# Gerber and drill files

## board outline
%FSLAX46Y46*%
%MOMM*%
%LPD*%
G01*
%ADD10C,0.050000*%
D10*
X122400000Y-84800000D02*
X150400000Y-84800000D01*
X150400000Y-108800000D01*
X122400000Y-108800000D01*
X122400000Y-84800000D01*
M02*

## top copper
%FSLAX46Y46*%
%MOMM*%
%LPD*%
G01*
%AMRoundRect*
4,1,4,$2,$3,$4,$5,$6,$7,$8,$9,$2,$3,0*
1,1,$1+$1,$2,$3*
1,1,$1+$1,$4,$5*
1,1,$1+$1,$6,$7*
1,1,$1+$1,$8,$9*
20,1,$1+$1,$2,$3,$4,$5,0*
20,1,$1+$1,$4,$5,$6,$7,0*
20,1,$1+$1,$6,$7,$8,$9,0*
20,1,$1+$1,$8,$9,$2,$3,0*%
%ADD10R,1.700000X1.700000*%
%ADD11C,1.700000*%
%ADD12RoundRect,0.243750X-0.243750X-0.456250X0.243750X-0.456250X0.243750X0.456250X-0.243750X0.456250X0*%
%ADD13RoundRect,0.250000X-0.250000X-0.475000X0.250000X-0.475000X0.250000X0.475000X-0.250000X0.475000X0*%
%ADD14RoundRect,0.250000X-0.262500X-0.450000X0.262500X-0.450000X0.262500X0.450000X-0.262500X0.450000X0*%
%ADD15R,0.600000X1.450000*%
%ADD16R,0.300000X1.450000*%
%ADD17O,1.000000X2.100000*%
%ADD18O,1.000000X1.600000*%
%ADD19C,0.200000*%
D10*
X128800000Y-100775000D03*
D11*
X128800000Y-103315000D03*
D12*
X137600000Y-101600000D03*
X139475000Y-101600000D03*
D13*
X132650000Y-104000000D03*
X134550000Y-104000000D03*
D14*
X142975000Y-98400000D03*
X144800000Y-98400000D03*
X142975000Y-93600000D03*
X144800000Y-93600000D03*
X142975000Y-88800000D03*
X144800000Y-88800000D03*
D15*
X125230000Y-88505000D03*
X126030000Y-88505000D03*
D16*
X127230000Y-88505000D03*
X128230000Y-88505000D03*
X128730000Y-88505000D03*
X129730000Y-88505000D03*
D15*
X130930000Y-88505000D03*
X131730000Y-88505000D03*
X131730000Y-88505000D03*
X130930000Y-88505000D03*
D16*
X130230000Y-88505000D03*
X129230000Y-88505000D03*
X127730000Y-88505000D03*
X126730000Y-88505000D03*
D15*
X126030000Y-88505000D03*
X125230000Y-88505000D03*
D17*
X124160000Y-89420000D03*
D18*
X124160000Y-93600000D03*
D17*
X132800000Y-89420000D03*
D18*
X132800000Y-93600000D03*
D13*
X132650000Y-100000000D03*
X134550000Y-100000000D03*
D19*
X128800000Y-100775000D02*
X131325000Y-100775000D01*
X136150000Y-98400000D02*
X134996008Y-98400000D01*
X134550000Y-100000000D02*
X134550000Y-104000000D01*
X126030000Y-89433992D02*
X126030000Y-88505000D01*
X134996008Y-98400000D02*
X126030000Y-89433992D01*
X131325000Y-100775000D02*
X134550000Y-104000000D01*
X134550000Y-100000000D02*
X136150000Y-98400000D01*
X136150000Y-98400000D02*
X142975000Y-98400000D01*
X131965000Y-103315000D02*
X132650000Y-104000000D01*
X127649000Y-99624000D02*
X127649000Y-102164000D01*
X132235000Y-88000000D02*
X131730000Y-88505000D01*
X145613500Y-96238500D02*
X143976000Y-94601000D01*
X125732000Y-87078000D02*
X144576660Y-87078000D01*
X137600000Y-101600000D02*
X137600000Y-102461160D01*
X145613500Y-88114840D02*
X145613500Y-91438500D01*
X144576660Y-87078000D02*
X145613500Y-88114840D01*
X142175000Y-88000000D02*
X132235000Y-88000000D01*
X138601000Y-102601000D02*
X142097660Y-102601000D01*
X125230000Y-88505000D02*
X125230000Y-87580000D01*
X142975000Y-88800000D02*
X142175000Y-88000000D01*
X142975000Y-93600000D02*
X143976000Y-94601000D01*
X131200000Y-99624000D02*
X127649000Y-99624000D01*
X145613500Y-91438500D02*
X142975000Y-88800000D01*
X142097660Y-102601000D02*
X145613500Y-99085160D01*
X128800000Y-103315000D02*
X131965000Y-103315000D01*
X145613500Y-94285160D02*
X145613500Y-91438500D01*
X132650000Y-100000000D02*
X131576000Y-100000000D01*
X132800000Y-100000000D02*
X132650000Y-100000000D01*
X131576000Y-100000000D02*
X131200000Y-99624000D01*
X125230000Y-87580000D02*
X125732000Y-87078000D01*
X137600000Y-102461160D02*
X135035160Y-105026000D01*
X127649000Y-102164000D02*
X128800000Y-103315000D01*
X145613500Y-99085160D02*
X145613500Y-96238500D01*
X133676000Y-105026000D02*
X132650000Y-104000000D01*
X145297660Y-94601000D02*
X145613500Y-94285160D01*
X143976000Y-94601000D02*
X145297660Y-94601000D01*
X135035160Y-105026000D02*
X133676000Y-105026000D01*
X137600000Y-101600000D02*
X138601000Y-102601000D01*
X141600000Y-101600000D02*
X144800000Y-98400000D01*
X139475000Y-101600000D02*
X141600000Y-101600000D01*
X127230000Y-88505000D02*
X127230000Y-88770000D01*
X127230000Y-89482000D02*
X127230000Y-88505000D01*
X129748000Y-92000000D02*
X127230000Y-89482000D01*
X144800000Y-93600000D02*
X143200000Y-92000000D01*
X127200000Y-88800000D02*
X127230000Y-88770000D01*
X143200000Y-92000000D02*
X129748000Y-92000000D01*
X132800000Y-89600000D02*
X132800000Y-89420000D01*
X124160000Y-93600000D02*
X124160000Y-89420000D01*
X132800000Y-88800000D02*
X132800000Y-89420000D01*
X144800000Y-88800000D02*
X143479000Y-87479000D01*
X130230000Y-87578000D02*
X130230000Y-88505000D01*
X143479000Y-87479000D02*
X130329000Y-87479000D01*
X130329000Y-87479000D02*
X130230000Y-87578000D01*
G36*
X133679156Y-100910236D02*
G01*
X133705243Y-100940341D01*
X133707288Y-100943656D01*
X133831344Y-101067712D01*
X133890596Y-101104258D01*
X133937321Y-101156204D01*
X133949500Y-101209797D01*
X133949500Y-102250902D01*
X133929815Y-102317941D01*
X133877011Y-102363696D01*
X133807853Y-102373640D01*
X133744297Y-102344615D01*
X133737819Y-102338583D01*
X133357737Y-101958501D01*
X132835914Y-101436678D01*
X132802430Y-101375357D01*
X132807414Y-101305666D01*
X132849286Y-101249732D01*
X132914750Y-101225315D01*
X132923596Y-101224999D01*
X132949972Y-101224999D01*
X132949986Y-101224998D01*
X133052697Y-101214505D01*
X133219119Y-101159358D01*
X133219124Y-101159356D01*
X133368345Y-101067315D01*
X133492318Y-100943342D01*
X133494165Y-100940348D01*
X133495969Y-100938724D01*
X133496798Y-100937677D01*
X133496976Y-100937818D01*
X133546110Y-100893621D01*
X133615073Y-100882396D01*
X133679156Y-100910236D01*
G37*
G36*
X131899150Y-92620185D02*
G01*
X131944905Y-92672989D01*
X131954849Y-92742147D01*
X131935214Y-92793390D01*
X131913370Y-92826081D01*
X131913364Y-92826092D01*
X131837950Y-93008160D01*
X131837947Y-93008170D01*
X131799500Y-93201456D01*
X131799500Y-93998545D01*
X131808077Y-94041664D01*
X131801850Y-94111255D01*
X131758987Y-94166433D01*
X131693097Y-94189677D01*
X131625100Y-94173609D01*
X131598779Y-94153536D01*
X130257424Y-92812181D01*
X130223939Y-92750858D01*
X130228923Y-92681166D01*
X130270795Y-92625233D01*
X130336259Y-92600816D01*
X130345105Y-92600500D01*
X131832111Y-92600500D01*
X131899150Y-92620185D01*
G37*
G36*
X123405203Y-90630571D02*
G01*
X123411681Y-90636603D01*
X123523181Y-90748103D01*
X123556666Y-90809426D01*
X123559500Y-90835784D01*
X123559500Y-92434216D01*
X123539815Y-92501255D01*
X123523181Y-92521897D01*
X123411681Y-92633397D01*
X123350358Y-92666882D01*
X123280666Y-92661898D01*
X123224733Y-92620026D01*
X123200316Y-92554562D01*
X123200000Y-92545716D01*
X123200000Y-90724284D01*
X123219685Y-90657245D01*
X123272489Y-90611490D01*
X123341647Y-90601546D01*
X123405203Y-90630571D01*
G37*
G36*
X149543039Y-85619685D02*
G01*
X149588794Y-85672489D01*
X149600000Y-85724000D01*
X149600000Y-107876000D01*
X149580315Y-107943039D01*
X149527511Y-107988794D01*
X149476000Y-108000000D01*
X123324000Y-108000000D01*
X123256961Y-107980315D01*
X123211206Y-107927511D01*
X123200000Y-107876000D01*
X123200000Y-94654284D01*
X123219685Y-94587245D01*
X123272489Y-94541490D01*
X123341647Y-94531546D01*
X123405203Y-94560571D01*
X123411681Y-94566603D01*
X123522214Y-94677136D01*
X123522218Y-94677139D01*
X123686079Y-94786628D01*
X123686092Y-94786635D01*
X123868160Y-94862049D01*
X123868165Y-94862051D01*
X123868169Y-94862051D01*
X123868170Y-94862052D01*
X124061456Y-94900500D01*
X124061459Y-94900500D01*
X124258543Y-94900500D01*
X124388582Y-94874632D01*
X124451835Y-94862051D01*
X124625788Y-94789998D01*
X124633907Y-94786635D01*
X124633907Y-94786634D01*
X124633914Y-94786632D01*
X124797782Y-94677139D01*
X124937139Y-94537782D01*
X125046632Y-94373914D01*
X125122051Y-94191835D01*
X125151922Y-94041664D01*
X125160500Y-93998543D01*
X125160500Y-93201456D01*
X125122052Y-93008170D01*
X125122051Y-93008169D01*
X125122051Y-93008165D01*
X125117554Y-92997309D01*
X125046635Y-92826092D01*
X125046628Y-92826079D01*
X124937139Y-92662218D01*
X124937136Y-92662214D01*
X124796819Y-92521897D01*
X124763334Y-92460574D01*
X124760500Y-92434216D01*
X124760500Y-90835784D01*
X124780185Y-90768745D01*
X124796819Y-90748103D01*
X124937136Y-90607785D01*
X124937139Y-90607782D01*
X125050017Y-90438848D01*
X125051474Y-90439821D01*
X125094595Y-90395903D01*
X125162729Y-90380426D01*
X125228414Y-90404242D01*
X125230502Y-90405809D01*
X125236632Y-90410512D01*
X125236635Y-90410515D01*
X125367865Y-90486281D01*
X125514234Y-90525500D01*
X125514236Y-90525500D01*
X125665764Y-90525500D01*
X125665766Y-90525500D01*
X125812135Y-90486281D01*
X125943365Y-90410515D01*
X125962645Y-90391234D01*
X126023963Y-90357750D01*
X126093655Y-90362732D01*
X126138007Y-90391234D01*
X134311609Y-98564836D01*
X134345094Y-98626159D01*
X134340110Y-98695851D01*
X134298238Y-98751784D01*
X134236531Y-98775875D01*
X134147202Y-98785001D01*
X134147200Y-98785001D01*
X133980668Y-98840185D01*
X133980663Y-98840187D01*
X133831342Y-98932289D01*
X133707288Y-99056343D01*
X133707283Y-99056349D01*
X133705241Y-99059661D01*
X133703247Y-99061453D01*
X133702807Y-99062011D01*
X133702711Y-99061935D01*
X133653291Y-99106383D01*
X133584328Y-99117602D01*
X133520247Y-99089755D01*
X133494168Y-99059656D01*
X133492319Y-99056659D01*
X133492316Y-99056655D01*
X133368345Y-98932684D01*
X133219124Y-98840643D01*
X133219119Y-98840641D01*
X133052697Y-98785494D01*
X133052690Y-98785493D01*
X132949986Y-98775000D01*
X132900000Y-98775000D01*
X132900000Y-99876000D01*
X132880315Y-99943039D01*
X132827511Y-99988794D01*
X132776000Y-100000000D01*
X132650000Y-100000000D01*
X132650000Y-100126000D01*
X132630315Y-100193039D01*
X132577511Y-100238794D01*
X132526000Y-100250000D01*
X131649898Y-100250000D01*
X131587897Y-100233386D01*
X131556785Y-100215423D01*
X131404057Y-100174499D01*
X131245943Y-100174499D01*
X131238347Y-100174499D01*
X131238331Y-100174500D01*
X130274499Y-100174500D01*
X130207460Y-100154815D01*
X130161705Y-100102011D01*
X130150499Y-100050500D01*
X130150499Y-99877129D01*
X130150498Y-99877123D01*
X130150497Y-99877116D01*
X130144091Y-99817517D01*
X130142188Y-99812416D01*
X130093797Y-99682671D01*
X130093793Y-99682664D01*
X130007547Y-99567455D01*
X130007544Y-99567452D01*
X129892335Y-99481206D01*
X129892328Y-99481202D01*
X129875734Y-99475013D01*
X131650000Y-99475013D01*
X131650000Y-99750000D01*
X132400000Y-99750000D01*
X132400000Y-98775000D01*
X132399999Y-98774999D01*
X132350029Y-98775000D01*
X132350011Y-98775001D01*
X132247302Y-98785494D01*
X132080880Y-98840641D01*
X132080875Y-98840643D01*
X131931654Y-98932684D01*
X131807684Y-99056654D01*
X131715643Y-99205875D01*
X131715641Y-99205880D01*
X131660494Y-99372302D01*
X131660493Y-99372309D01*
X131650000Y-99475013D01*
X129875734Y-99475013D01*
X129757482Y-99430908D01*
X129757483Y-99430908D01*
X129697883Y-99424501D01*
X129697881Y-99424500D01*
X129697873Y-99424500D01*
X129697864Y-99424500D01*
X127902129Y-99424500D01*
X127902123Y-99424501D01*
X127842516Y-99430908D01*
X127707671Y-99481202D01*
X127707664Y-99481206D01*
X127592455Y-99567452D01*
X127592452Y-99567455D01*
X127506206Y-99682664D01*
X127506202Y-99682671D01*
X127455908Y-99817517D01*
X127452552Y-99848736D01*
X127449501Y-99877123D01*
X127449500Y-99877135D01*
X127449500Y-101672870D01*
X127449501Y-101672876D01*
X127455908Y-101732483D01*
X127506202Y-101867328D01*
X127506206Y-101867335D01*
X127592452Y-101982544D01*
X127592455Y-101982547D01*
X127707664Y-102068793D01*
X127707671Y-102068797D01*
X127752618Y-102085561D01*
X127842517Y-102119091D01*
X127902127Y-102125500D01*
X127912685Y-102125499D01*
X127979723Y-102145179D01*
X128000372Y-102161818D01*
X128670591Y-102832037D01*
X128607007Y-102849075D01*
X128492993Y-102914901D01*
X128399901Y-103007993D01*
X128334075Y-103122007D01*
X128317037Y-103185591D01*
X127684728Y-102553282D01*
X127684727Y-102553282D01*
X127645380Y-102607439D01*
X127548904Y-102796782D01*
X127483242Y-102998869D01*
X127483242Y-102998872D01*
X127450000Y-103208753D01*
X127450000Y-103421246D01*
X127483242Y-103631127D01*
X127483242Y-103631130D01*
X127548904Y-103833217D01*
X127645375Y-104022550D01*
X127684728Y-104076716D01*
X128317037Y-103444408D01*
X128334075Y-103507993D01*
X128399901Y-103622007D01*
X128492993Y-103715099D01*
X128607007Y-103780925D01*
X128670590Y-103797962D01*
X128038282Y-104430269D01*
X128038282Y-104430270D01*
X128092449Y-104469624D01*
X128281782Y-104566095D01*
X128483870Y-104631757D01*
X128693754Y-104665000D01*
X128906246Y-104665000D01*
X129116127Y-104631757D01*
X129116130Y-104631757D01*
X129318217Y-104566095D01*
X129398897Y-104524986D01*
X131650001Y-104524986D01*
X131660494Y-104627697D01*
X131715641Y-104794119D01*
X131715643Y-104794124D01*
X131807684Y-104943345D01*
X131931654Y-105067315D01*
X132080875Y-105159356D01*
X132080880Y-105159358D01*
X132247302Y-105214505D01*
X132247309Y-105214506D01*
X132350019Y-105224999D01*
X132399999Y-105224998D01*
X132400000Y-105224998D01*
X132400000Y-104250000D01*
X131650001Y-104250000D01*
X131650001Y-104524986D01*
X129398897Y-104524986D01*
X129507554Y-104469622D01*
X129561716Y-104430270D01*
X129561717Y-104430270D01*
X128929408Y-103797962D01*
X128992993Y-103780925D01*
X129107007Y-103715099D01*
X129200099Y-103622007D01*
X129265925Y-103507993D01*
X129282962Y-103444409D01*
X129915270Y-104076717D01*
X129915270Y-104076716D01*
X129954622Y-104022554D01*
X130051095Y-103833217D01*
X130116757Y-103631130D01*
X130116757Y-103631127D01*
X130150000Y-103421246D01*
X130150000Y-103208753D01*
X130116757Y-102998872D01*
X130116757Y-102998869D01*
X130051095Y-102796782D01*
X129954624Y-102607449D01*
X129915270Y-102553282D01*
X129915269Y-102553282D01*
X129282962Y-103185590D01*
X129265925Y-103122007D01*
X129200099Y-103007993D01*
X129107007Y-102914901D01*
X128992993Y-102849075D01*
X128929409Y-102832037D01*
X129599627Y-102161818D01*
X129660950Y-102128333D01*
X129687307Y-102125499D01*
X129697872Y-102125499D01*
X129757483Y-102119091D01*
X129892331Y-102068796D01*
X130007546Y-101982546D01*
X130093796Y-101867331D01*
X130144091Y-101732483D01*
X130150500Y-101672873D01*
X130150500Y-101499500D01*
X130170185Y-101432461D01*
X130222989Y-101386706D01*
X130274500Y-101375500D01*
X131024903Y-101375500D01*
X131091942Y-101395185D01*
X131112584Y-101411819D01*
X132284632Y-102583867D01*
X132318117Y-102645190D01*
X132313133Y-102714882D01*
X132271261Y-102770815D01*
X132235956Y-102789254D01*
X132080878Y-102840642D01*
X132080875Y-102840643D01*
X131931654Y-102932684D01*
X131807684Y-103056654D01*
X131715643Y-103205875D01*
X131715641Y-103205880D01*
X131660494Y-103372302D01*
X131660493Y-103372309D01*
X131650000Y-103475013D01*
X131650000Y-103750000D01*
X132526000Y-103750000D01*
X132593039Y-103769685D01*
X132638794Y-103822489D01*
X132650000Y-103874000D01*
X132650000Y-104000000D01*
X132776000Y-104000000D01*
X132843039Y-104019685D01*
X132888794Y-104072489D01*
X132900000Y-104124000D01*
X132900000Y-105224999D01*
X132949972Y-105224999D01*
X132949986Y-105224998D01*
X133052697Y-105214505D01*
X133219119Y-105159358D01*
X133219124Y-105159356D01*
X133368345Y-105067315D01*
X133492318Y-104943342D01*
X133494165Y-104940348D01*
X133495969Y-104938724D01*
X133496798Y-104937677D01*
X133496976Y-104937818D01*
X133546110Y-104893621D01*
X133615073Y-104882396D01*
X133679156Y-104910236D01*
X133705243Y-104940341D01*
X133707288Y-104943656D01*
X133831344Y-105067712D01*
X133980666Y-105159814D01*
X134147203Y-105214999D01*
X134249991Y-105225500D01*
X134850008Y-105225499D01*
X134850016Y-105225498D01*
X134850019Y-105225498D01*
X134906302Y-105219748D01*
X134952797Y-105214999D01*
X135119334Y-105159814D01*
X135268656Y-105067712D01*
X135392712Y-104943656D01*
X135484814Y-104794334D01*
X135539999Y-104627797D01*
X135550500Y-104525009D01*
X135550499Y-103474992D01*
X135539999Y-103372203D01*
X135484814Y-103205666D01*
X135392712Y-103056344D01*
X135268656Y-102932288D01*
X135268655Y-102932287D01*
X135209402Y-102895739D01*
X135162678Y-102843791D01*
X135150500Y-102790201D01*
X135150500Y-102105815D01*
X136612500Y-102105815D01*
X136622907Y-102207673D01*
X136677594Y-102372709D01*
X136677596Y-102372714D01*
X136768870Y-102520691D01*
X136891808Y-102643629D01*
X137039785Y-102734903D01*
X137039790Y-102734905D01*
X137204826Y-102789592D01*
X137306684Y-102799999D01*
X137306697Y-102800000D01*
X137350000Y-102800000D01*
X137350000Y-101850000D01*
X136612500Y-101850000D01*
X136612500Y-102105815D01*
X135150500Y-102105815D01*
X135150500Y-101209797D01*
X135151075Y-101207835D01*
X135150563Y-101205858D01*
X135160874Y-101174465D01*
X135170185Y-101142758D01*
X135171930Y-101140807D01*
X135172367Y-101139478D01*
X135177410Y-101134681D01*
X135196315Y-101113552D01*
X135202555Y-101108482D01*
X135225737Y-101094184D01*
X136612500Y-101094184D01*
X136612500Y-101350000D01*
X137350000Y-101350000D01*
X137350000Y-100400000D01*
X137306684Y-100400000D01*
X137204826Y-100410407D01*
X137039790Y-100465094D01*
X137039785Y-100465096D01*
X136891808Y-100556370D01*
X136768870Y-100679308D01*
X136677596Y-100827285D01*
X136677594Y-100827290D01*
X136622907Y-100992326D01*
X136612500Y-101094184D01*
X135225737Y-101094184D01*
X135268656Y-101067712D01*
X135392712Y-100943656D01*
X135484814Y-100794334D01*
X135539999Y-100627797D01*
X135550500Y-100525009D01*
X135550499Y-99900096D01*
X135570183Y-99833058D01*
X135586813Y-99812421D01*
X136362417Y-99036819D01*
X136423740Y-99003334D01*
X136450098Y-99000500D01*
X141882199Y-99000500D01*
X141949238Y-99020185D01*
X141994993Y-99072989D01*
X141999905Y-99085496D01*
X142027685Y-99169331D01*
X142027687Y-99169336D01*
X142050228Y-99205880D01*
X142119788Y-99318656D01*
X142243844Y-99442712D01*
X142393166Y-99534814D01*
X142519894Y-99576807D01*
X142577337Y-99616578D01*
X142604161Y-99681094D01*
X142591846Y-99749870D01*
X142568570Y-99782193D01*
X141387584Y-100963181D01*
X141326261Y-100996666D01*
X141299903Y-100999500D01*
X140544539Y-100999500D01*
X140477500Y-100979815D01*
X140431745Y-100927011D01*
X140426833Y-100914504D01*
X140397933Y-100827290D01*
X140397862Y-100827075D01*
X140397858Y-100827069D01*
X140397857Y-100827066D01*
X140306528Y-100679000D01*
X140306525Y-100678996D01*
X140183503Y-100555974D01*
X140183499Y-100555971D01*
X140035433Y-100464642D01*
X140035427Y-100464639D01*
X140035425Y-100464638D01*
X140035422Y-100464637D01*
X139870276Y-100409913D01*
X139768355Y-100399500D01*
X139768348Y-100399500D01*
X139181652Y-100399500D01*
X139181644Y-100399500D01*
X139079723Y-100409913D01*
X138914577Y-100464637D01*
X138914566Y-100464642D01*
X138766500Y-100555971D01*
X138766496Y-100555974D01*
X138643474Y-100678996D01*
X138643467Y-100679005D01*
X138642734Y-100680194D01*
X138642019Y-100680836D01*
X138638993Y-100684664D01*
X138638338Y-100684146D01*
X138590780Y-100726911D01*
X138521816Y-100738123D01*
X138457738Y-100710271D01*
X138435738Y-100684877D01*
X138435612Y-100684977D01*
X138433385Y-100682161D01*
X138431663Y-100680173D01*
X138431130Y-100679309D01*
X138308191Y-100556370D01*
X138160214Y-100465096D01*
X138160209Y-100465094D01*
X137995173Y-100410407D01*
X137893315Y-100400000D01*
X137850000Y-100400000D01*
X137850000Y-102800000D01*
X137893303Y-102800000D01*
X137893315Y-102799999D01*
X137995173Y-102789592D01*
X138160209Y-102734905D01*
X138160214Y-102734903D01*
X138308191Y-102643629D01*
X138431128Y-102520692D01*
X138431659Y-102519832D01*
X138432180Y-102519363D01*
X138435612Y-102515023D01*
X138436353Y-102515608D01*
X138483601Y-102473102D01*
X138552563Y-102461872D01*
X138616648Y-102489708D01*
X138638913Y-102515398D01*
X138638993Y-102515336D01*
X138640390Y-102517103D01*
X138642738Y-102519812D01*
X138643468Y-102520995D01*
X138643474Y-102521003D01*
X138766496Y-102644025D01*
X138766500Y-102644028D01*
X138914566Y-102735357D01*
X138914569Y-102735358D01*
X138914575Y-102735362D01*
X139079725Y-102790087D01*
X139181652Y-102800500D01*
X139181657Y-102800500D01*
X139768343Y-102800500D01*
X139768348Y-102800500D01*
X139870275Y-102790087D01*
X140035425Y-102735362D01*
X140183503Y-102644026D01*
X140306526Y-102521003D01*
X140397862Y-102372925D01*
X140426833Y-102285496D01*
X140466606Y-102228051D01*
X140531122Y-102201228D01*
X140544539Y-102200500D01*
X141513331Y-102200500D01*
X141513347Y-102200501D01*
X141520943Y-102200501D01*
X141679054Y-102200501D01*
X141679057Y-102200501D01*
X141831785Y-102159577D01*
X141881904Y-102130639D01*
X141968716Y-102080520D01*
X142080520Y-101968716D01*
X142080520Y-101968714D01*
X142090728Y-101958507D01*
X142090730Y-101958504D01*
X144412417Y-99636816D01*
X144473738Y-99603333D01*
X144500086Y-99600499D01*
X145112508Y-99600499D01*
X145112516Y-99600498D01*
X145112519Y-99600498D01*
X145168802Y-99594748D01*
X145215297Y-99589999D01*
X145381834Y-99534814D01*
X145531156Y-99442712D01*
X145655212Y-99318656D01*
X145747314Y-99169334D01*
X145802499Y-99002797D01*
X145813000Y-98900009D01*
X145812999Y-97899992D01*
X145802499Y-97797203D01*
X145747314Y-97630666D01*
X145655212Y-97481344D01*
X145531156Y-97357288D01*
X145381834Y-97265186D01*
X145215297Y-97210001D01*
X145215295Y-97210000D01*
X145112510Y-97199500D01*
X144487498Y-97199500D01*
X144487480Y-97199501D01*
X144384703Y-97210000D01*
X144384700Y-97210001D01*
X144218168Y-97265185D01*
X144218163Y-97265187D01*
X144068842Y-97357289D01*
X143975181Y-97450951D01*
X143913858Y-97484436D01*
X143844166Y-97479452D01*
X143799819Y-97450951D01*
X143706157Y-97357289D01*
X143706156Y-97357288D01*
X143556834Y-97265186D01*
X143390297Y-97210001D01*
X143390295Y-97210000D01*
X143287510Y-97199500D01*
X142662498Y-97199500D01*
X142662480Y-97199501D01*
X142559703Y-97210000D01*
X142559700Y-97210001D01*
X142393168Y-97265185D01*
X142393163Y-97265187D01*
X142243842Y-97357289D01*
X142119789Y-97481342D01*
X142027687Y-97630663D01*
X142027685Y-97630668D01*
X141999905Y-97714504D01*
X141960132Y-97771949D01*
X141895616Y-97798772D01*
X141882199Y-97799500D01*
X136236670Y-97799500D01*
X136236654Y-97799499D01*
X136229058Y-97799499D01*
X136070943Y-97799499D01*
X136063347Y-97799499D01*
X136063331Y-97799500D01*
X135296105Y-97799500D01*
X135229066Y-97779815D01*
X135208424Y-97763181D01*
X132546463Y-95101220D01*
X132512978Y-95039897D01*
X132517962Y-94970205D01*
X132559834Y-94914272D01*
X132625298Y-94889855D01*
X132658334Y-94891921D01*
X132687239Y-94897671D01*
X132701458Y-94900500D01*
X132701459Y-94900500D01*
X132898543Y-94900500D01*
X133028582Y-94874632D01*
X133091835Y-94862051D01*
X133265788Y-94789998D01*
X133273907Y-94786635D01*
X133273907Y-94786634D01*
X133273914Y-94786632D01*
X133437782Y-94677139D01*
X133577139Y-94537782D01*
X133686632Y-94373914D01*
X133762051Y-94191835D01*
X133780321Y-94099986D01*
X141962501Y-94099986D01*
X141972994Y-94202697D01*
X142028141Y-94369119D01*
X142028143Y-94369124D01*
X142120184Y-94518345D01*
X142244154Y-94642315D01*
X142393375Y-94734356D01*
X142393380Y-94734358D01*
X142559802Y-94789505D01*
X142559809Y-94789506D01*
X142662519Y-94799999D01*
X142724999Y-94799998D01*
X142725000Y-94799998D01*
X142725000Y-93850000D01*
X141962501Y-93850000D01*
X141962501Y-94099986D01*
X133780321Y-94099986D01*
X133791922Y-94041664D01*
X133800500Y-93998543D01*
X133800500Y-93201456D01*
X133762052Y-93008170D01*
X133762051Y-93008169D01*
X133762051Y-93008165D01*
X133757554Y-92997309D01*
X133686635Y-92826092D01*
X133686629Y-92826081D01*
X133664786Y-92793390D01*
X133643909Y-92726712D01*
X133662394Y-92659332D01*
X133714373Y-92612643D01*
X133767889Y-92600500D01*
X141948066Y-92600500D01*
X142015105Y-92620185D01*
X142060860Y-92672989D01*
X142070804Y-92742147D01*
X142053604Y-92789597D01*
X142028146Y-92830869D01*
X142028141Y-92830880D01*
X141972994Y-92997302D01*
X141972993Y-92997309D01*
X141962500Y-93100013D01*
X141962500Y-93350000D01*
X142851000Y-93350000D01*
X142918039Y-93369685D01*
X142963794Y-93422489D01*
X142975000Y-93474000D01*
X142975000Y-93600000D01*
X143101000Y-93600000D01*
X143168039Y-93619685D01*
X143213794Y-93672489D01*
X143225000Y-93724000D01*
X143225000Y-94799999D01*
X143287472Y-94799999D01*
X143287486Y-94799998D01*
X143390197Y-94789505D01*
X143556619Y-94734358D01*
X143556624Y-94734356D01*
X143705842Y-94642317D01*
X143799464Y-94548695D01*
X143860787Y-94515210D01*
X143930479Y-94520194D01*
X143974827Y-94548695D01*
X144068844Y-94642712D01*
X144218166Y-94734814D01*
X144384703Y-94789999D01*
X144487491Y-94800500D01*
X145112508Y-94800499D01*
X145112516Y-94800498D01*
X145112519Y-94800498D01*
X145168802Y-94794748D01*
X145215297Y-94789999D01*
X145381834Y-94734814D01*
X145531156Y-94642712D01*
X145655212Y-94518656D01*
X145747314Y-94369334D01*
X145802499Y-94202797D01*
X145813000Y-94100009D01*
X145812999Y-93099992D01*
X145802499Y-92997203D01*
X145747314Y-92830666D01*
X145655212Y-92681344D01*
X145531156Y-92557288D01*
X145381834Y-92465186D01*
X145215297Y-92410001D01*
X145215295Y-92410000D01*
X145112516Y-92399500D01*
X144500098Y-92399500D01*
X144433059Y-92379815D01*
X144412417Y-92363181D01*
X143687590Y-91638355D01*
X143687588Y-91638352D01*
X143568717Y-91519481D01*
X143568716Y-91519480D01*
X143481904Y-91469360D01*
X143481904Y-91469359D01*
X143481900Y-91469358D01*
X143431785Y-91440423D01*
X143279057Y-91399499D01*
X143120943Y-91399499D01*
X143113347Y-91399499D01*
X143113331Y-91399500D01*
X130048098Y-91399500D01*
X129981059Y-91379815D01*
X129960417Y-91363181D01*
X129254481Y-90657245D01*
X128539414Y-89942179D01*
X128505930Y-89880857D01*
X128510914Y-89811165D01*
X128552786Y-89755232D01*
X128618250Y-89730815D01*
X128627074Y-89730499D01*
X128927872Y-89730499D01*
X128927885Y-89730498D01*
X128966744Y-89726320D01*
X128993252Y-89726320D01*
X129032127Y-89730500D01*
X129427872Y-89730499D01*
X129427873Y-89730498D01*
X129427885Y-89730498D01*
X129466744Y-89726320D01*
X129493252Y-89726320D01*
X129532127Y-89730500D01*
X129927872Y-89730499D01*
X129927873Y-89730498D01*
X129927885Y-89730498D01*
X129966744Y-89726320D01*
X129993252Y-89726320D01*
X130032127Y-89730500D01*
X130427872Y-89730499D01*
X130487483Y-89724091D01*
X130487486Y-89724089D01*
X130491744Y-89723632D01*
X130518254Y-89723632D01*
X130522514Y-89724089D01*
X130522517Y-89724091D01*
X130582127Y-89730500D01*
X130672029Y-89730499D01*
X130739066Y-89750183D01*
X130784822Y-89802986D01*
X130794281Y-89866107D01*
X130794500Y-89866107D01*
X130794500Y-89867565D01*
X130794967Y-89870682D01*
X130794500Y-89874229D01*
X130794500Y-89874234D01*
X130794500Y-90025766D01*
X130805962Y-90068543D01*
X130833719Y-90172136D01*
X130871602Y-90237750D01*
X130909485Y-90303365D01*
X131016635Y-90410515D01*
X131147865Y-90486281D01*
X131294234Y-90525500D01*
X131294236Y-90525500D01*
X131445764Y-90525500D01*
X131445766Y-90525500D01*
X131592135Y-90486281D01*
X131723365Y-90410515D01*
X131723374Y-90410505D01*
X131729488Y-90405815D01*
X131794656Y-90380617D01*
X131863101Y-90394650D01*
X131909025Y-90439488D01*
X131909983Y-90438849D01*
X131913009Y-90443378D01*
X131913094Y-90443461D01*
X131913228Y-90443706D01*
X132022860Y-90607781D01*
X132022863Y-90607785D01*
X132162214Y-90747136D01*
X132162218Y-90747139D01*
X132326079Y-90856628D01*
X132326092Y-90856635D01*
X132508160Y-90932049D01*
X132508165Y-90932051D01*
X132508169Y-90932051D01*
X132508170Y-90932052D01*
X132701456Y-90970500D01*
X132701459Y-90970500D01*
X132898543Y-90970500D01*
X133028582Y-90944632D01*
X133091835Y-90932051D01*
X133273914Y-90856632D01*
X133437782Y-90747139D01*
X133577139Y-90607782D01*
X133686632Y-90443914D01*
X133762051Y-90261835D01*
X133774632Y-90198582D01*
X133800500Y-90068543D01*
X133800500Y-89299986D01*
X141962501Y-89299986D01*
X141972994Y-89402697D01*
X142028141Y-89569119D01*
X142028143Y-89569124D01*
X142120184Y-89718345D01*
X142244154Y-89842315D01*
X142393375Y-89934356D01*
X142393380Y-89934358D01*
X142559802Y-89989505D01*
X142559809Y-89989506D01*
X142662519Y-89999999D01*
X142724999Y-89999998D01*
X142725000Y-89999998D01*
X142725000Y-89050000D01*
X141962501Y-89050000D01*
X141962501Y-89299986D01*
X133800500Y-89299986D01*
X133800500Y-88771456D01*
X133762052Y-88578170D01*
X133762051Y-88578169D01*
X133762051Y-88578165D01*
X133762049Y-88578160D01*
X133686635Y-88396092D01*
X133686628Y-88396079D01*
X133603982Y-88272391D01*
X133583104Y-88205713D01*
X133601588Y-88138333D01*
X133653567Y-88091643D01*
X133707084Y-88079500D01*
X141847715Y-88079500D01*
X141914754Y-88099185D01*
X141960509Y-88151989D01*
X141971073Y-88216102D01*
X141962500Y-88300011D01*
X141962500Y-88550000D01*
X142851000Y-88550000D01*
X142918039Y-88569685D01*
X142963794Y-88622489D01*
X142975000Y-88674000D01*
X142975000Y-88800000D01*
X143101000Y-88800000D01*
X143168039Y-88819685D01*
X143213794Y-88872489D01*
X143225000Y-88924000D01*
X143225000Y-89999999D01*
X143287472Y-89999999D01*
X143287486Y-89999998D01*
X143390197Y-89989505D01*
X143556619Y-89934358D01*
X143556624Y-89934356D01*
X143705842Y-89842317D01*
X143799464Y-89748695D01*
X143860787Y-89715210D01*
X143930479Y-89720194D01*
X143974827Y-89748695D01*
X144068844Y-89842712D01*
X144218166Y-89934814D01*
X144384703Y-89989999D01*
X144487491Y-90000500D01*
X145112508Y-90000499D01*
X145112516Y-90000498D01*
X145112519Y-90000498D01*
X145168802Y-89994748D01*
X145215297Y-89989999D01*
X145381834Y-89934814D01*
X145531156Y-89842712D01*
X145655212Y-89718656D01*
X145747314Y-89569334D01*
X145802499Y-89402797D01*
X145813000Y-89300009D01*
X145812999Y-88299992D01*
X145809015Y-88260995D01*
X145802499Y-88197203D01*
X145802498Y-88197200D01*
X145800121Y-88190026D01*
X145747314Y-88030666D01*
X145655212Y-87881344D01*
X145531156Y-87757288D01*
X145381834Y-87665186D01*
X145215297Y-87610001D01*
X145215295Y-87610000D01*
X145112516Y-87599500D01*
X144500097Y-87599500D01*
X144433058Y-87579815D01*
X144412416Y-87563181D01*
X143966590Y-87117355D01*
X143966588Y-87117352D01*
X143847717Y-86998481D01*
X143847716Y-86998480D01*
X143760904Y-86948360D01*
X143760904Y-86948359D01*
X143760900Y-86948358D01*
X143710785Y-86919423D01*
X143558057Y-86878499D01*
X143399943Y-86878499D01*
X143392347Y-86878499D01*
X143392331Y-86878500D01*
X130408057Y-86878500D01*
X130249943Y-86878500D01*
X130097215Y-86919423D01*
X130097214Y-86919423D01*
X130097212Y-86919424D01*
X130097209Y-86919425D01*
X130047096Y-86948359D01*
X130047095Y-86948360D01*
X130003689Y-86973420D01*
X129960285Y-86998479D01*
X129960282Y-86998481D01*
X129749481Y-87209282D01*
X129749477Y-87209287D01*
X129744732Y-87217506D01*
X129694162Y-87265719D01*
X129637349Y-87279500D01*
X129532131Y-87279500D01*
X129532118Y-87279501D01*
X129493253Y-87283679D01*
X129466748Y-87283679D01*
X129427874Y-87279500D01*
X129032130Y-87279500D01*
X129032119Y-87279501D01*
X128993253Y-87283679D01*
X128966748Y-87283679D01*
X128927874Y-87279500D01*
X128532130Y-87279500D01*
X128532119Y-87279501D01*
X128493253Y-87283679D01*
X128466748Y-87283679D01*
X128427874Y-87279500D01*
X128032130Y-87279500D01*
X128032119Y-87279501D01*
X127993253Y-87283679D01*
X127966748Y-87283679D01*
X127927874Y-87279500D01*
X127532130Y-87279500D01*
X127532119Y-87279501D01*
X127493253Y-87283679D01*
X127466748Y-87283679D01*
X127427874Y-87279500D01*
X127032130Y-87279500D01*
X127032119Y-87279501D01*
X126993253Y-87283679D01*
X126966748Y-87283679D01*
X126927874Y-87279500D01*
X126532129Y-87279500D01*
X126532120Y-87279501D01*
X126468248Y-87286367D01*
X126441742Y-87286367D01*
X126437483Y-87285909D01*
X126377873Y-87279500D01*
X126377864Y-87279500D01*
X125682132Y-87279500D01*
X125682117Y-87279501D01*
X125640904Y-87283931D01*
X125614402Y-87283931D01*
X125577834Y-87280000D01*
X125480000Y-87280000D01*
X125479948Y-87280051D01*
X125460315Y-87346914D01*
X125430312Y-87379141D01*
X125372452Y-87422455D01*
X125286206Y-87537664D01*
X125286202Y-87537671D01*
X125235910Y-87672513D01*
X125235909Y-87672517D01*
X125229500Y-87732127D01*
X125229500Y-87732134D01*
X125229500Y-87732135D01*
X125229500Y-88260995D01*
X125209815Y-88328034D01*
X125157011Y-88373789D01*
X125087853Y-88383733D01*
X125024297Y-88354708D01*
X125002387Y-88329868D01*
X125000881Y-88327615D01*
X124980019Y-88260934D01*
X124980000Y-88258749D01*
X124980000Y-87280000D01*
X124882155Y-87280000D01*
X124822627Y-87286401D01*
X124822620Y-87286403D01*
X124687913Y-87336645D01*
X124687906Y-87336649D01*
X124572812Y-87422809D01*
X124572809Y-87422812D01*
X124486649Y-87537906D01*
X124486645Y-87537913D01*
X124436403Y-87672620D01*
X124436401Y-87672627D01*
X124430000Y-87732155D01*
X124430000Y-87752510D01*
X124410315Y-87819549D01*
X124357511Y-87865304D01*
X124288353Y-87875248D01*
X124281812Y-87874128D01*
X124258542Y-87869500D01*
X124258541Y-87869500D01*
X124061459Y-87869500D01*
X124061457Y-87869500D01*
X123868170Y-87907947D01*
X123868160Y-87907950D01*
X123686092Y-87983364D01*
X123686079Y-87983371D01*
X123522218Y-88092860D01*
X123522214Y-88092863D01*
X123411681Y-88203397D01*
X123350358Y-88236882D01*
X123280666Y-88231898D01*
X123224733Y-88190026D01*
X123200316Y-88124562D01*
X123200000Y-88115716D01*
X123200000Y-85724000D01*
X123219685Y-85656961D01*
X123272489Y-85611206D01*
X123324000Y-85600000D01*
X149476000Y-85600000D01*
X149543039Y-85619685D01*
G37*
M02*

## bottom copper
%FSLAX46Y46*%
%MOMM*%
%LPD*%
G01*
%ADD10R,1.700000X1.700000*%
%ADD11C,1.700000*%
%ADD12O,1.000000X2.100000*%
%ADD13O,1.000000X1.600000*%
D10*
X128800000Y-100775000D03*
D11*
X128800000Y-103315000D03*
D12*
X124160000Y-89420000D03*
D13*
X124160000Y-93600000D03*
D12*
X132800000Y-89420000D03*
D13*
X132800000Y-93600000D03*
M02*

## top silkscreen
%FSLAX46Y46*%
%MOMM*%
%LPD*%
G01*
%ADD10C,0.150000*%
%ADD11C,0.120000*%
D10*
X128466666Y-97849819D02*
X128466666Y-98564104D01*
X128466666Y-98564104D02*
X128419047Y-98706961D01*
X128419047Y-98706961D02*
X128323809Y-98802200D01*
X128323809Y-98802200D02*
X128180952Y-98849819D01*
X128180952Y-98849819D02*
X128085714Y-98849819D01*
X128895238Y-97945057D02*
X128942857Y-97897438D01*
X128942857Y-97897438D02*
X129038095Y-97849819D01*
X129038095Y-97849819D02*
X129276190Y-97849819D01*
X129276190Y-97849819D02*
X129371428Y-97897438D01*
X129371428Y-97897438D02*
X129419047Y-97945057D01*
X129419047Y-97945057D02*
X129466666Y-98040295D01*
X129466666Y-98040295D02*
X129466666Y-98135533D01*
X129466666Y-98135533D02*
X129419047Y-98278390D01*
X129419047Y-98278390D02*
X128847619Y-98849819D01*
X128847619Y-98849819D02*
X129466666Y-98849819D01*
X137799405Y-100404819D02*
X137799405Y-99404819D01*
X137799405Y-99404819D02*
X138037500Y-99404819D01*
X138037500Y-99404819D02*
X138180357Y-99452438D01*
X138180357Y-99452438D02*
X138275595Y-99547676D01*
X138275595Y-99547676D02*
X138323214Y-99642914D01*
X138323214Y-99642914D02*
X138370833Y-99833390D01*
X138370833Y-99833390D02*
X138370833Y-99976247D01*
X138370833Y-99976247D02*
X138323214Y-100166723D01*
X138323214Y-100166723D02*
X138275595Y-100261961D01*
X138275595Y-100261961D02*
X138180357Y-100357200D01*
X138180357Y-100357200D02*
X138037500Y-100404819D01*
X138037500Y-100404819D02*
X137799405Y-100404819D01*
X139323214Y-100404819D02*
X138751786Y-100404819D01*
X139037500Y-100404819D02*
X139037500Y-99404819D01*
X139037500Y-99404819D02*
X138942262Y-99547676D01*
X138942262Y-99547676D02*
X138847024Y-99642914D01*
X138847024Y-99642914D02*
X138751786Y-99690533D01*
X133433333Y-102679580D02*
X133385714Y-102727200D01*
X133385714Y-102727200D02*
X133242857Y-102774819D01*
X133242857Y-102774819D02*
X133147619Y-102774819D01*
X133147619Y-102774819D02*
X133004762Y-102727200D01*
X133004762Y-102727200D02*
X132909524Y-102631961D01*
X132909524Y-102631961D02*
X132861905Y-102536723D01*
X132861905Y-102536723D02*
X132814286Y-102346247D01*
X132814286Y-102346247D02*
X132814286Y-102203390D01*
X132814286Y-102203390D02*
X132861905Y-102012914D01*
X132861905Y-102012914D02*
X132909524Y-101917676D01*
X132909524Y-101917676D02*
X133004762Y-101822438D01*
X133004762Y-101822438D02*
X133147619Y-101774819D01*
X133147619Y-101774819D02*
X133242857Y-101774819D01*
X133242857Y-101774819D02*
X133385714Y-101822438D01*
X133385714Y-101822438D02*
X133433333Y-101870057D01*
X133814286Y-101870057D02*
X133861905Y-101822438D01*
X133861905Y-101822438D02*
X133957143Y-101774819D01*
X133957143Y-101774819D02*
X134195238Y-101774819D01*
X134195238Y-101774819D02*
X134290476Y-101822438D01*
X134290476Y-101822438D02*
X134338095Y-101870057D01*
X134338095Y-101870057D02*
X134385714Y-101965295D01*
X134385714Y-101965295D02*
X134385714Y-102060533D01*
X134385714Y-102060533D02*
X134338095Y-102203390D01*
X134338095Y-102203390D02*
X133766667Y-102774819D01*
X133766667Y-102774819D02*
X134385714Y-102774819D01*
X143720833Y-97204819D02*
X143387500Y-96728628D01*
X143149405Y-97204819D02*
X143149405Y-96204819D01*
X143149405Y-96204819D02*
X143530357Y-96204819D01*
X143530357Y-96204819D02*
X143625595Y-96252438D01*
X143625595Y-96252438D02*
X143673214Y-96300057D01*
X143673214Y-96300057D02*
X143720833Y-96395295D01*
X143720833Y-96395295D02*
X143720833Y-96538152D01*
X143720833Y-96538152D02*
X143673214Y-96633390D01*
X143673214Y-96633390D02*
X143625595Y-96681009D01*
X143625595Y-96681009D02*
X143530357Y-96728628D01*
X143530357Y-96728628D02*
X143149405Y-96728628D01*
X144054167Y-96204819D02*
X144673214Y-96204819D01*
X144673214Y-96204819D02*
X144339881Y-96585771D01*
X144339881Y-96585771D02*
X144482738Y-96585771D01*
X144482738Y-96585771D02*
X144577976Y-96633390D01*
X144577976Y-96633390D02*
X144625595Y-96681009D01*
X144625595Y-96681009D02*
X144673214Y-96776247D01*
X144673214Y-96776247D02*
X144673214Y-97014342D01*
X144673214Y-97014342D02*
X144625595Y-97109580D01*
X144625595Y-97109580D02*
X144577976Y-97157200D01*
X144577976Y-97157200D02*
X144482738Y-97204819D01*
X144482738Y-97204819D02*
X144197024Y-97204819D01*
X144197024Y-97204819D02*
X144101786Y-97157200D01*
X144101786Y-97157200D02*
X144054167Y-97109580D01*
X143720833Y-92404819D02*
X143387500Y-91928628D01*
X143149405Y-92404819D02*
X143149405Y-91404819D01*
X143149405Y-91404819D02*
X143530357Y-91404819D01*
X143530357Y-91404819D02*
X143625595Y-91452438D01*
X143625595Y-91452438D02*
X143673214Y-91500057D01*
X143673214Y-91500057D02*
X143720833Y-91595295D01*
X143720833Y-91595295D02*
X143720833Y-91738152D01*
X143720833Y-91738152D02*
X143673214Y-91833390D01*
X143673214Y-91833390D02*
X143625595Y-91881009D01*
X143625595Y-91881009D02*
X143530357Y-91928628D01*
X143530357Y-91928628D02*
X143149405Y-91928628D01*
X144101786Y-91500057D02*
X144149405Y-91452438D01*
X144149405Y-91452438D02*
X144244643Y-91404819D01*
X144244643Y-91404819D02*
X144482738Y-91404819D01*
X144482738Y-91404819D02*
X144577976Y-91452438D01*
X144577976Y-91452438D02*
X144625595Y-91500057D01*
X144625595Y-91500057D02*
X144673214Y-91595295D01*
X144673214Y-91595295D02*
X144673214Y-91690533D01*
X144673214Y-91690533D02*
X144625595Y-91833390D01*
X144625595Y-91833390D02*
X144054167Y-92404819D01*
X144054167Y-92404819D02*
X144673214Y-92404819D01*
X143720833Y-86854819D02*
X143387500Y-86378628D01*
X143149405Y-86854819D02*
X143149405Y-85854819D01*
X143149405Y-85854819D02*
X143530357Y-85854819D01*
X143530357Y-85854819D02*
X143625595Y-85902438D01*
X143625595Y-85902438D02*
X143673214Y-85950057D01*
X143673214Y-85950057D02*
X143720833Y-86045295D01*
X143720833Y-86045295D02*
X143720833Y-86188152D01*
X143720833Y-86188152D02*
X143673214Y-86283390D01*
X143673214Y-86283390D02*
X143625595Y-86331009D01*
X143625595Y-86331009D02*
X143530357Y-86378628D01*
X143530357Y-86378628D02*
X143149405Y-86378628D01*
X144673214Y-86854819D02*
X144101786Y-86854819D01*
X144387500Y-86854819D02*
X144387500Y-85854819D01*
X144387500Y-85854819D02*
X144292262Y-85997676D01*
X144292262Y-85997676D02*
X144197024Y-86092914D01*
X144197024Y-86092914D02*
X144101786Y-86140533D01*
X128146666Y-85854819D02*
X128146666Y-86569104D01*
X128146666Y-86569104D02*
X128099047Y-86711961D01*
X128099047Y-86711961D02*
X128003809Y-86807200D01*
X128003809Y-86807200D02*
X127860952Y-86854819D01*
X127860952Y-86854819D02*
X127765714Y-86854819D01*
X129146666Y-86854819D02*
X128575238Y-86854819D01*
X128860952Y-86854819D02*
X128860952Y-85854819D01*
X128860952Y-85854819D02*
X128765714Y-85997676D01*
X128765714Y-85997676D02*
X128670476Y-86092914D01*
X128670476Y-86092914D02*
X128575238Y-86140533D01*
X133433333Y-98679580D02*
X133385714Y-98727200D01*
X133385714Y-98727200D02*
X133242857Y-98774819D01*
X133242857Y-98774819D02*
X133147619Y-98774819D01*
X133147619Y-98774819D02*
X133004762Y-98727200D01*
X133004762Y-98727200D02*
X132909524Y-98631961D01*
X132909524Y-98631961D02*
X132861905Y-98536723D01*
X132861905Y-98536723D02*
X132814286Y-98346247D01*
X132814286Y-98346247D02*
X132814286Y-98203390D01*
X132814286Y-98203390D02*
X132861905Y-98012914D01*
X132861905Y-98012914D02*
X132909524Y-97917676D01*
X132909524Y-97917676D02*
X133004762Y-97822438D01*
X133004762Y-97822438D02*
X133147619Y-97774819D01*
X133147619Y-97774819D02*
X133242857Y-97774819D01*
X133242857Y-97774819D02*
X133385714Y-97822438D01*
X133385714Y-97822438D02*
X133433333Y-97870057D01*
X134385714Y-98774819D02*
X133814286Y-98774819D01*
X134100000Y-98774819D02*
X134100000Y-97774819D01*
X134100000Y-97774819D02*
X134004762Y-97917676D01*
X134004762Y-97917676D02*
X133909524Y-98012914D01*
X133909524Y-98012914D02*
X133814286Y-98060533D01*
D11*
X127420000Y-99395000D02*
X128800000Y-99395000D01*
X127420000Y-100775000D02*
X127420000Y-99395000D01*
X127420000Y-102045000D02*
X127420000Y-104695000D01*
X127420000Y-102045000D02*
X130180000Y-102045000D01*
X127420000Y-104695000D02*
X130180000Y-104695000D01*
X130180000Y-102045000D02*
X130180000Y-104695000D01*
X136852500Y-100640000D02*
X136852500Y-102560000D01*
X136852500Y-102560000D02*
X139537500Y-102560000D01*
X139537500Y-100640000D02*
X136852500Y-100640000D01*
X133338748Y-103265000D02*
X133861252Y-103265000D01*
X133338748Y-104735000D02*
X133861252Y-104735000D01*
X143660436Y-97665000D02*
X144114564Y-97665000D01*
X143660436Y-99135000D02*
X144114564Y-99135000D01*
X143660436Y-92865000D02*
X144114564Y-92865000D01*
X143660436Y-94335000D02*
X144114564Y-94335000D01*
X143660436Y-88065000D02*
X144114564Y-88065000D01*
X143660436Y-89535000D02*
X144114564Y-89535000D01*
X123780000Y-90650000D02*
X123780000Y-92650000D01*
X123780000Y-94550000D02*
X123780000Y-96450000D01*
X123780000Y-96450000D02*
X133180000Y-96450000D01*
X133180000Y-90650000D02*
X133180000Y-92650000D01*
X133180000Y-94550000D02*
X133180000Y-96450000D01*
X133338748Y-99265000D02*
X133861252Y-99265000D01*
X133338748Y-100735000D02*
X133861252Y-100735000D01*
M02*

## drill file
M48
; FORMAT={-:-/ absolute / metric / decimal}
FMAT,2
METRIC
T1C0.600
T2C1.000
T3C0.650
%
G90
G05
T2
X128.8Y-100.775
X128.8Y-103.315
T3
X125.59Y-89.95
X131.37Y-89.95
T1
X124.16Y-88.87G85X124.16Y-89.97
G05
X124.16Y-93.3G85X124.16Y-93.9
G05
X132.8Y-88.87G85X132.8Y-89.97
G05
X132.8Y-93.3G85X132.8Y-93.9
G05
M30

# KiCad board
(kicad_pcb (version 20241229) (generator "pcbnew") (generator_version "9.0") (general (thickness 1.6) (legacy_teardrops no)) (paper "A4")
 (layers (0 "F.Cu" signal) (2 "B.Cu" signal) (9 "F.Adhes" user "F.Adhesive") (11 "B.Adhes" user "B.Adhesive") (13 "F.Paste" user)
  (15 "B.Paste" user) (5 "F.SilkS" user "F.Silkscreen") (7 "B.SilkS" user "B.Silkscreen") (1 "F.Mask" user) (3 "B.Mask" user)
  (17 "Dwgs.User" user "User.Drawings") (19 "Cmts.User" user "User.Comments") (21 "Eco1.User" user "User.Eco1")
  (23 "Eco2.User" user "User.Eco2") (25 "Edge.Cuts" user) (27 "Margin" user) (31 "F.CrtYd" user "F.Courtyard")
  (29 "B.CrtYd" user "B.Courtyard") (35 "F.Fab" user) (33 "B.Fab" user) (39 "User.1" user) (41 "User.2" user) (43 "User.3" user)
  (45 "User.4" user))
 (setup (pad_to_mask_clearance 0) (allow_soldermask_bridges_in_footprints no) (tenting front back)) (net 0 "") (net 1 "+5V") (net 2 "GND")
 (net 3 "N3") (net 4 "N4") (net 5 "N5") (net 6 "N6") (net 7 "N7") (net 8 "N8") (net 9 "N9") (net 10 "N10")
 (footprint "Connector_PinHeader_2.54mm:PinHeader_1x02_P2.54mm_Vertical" (layer "F.Cu") (at 128.8 100.775)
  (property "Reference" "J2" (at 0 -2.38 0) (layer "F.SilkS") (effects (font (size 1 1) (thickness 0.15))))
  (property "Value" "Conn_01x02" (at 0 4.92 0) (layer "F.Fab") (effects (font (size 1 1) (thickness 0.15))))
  (fp_line (start -1.38 -1.38) (end 0 -1.38) (stroke (width 0.12) (type solid)) (layer "F.SilkS"))
  (fp_line (start -1.38 0) (end -1.38 -1.38) (stroke (width 0.12) (type solid)) (layer "F.SilkS"))
  (fp_line (start -1.38 1.27) (end -1.38 3.92) (stroke (width 0.12) (type solid)) (layer "F.SilkS"))
  (fp_line (start -1.38 1.27) (end 1.38 1.27) (stroke (width 0.12) (type solid)) (layer "F.SilkS"))
  (fp_line (start -1.38 3.92) (end 1.38 3.92) (stroke (width 0.12) (type solid)) (layer "F.SilkS"))
  (fp_line (start 1.38 1.27) (end 1.38 3.92) (stroke (width 0.12) (type solid)) (layer "F.SilkS"))
  (pad "1" thru_hole rect (at 0 0) (size 1.7 1.7) (drill 1) (layers "*.Cu" "*.Mask") (remove_unused_layers no) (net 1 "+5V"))
  (pad "2" thru_hole circle (at 0 2.54) (size 1.7 1.7) (drill 1) (layers "*.Cu" "*.Mask") (remove_unused_layers no) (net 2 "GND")))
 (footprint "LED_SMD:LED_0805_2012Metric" (layer "F.Cu") (at 138.5375 101.6)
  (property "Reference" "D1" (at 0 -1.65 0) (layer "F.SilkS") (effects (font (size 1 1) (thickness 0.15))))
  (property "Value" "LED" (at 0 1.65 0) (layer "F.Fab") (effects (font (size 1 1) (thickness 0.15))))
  (fp_line (start -1.685 -0.96) (end -1.685 0.96) (stroke (width 0.12) (type solid)) (layer "F.SilkS"))
  (fp_line (start -1.685 0.96) (end 1 0.96) (stroke (width 0.12) (type solid)) (layer "F.SilkS"))
  (fp_line (start 1 -0.96) (end -1.685 -0.96) (stroke (width 0.12) (type solid)) (layer "F.SilkS"))
  (pad "1" smd roundrect (at -0.9375 0) (size 0.975 1.4) (layers "F.Cu" "F.Mask" "F.Paste") (roundrect_rratio 0.25) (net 2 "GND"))
  (pad "2" smd roundrect (at 0.9375 0) (size 0.975 1.4) (layers "F.Cu" "F.Mask" "F.Paste") (roundrect_rratio 0.25) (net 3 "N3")))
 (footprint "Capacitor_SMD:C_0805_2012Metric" (layer "F.Cu") (at 133.6 104)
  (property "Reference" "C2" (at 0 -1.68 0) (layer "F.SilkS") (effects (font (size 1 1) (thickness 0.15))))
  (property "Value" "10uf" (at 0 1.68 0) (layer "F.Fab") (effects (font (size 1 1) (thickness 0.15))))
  (fp_line (start -0.261252 -0.735) (end 0.261252 -0.735) (stroke (width 0.12) (type solid)) (layer "F.SilkS"))
  (fp_line (start -0.261252 0.735) (end 0.261252 0.735) (stroke (width 0.12) (type solid)) (layer "F.SilkS"))
  (pad "1" smd roundrect (at -0.95 0) (size 1 1.45) (layers "F.Cu" "F.Mask" "F.Paste") (roundrect_rratio 0.25) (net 2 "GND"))
  (pad "2" smd roundrect (at 0.95 0) (size 1 1.45) (layers "F.Cu" "F.Mask" "F.Paste") (roundrect_rratio 0.25) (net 1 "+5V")))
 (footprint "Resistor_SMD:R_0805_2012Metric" (layer "F.Cu") (at 143.8875 98.4)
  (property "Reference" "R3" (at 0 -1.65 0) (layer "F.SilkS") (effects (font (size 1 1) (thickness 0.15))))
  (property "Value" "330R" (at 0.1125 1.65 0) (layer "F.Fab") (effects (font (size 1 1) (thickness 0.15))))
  (fp_line (start -0.227064 -0.735) (end 0.227064 -0.735) (stroke (width 0.12) (type solid)) (layer "F.SilkS"))
  (fp_line (start -0.227064 0.735) (end 0.227064 0.735) (stroke (width 0.12) (type solid)) (layer "F.SilkS"))
  (pad "1" smd roundrect (at -0.9125 0) (size 1.025 1.4) (layers "F.Cu" "F.Mask" "F.Paste") (roundrect_rratio 0.243902) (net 1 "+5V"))
  (pad "2" smd roundrect (at 0.9125 0) (size 1.025 1.4) (layers "F.Cu" "F.Mask" "F.Paste") (roundrect_rratio 0.243902) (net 3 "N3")))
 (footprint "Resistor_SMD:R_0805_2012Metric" (layer "F.Cu") (at 143.8875 93.6)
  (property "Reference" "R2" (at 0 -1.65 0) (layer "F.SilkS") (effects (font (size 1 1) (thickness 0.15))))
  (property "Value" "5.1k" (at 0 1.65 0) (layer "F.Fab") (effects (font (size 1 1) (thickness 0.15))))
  (fp_line (start -0.227064 -0.735) (end 0.227064 -0.735) (stroke (width 0.12) (type solid)) (layer "F.SilkS"))
  (fp_line (start -0.227064 0.735) (end 0.227064 0.735) (stroke (width 0.12) (type solid)) (layer "F.SilkS"))
  (pad "1" smd roundrect (at -0.9125 0) (size 1.025 1.4) (layers "F.Cu" "F.Mask" "F.Paste") (roundrect_rratio 0.243902) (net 2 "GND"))
  (pad "2" smd roundrect (at 0.9125 0) (size 1.025 1.4) (layers "F.Cu" "F.Mask" "F.Paste") (roundrect_rratio 0.243902) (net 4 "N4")))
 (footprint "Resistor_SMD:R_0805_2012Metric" (layer "F.Cu") (at 143.8875 88.8)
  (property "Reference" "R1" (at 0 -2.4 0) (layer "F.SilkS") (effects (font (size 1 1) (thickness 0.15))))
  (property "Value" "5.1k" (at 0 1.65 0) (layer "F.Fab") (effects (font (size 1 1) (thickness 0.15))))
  (fp_line (start -0.227064 -0.735) (end 0.227064 -0.735) (stroke (width 0.12) (type solid)) (layer "F.SilkS"))
  (fp_line (start -0.227064 0.735) (end 0.227064 0.735) (stroke (width 0.12) (type solid)) (layer "F.SilkS"))
  (pad "1" smd roundrect (at -0.9125 0) (size 1.025 1.4) (layers "F.Cu" "F.Mask" "F.Paste") (roundrect_rratio 0.243902) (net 2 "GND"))
  (pad "2" smd roundrect (at 0.9125 0) (size 1.025 1.4) (layers "F.Cu" "F.Mask" "F.Paste") (roundrect_rratio 0.243902) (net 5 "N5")))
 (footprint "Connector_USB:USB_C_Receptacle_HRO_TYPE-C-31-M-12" (layer "F.Cu") (at 128.48 92.55)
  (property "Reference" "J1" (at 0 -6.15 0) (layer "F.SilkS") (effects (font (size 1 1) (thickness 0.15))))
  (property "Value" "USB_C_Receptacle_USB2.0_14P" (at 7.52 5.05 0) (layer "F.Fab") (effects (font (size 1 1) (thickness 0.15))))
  (fp_line (start -4.7 -1.9) (end -4.7 0.1) (stroke (width 0.12) (type solid)) (layer "F.SilkS"))
  (fp_line (start -4.7 2) (end -4.7 3.9) (stroke (width 0.12) (type solid)) (layer "F.SilkS"))
  (fp_line (start -4.7 3.9) (end 4.7 3.9) (stroke (width 0.12) (type solid)) (layer "F.SilkS"))
  (fp_line (start 4.7 -1.9) (end 4.7 0.1) (stroke (width 0.12) (type solid)) (layer "F.SilkS"))
  (fp_line (start 4.7 2) (end 4.7 3.9) (stroke (width 0.12) (type solid)) (layer "F.SilkS"))
  (pad "" np_thru_hole circle (at -2.89 -2.6) (size 0.65 0.65) (drill 0.65) (layers "*.Cu" "*.Mask"))
  (pad "" np_thru_hole circle (at 2.89 -2.6) (size 0.65 0.65) (drill 0.65) (layers "*.Cu" "*.Mask"))
  (pad "A1" smd rect (at -3.25 -4.045) (size 0.6 1.45) (layers "F.Cu" "F.Mask" "F.Paste") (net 2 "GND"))
  (pad "A4" smd rect (at -2.45 -4.045) (size 0.6 1.45) (layers "F.Cu" "F.Mask" "F.Paste") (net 1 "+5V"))
  (pad "A5" smd rect (at -1.25 -4.045) (size 0.3 1.45) (layers "F.Cu" "F.Mask" "F.Paste") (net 4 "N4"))
  (pad "A6" smd rect (at -0.25 -4.045) (size 0.3 1.45) (layers "F.Cu" "F.Mask" "F.Paste") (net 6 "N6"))
  (pad "A7" smd rect (at 0.25 -4.045) (size 0.3 1.45) (layers "F.Cu" "F.Mask" "F.Paste") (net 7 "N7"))
  (pad "A8" smd rect (at 1.25 -4.045) (size 0.3 1.45) (layers "F.Cu" "F.Mask" "F.Paste"))
  (pad "A9" smd rect (at 2.45 -4.045) (size 0.6 1.45) (layers "F.Cu" "F.Mask" "F.Paste") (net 1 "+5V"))
  (pad "A12" smd rect (at 3.25 -4.045) (size 0.6 1.45) (layers "F.Cu" "F.Mask" "F.Paste") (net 2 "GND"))
  (pad "B1" smd rect (at 3.25 -4.045) (size 0.6 1.45) (layers "F.Cu" "F.Mask" "F.Paste") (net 2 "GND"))
  (pad "B4" smd rect (at 2.45 -4.045) (size 0.6 1.45) (layers "F.Cu" "F.Mask" "F.Paste") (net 1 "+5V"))
  (pad "B5" smd rect (at 1.75 -4.045) (size 0.3 1.45) (layers "F.Cu" "F.Mask" "F.Paste") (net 5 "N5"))
  (pad "B6" smd rect (at 0.75 -4.045) (size 0.3 1.45) (layers "F.Cu" "F.Mask" "F.Paste") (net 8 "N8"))
  (pad "B7" smd rect (at -0.75 -4.045) (size 0.3 1.45) (layers "F.Cu" "F.Mask" "F.Paste") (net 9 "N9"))
  (pad "B8" smd rect (at -1.75 -4.045) (size 0.3 1.45) (layers "F.Cu" "F.Mask" "F.Paste"))
  (pad "B9" smd rect (at -2.45 -4.045) (size 0.6 1.45) (layers "F.Cu" "F.Mask" "F.Paste") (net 1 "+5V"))
  (pad "B12" smd rect (at -3.25 -4.045) (size 0.6 1.45) (layers "F.Cu" "F.Mask" "F.Paste") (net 2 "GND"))
  (pad "S1" thru_hole oval (at -4.32 -3.13) (size 1 2.1) (drill oval 0.6 1.7) (layers "*.Cu" "*.Mask") (remove_unused_layers no)
   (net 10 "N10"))
  (pad "S1" thru_hole oval (at -4.32 1.05) (size 1 1.6) (drill oval 0.6 1.2) (layers "*.Cu" "*.Mask") (remove_unused_layers no)
   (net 10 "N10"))
  (pad "S1" thru_hole oval (at 4.32 -3.13) (size 1 2.1) (drill oval 0.6 1.7) (layers "*.Cu" "*.Mask") (remove_unused_layers no)
   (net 10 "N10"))
  (pad "S1" thru_hole oval (at 4.32 1.05) (size 1 1.6) (drill oval 0.6 1.2) (layers "*.Cu" "*.Mask") (remove_unused_layers no)
   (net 10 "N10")))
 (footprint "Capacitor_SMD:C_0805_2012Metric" (layer "F.Cu") (at 133.6 100)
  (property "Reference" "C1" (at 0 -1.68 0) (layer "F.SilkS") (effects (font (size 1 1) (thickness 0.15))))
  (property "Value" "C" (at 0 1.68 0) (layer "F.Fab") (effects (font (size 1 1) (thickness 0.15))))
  (fp_line (start -0.261252 -0.735) (end 0.261252 -0.735) (stroke (width 0.12) (type solid)) (layer "F.SilkS"))
  (fp_line (start -0.261252 0.735) (end 0.261252 0.735) (stroke (width 0.12) (type solid)) (layer "F.SilkS"))
  (pad "1" smd roundrect (at -0.95 0) (size 1 1.45) (layers "F.Cu" "F.Mask" "F.Paste") (roundrect_rratio 0.25) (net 2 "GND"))
  (pad "2" smd roundrect (at 0.95 0) (size 1 1.45) (layers "F.Cu" "F.Mask" "F.Paste") (roundrect_rratio 0.25) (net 1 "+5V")))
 (gr_rect (start 122.4 84.8) (end 150.4 108.8) (stroke (width 0.05) (type default)) (fill no) (layer "Edge.Cuts"))
 (segment (start 128.8 100.775) (end 131.325 100.775) (width 0.2) (layer "F.Cu") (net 1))
 (segment (start 136.15 98.4) (end 134.996008 98.4) (width 0.2) (layer "F.Cu") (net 1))
 (segment (start 134.55 100) (end 134.55 104) (width 0.2) (layer "F.Cu") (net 1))
 (segment (start 126.03 89.433992) (end 126.03 88.505) (width 0.2) (layer "F.Cu") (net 1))
 (segment (start 134.996008 98.4) (end 126.03 89.433992) (width 0.2) (layer "F.Cu") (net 1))
 (segment (start 131.325 100.775) (end 134.55 104) (width 0.2) (layer "F.Cu") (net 1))
 (segment (start 134.55 100) (end 136.15 98.4) (width 0.2) (layer "F.Cu") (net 1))
 (segment (start 136.15 98.4) (end 142.975 98.4) (width 0.2) (layer "F.Cu") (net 1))
 (segment (start 131.965 103.315) (end 132.65 104) (width 0.2) (layer "F.Cu") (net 2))
 (segment (start 127.649 99.624) (end 127.649 102.164) (width 0.2) (layer "F.Cu") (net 2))
 (segment (start 132.235 88) (end 131.73 88.505) (width 0.2) (layer "F.Cu") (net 2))
 (segment (start 145.6135 96.2385) (end 143.976 94.601) (width 0.2) (layer "F.Cu") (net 2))
 (segment (start 125.732 87.078) (end 144.57666 87.078) (width 0.2) (layer "F.Cu") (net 2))
 (segment (start 137.6 101.6) (end 137.6 102.46116) (width 0.2) (layer "F.Cu") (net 2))
 (segment (start 145.6135 88.11484) (end 145.6135 91.4385) (width 0.2) (layer "F.Cu") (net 2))
 (segment (start 144.57666 87.078) (end 145.6135 88.11484) (width 0.2) (layer "F.Cu") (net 2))
 (segment (start 142.175 88) (end 132.235 88) (width 0.2) (layer "F.Cu") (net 2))
 (segment (start 138.601 102.601) (end 142.09766 102.601) (width 0.2) (layer "F.Cu") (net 2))
 (segment (start 125.23 88.505) (end 125.23 87.58) (width 0.2) (layer "F.Cu") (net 2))
 (segment (start 142.975 88.8) (end 142.175 88) (width 0.2) (layer "F.Cu") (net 2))
 (segment (start 142.975 93.6) (end 143.976 94.601) (width 0.2) (layer "F.Cu") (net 2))
 (segment (start 131.2 99.624) (end 127.649 99.624) (width 0.2) (layer "F.Cu") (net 2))
 (segment (start 145.6135 91.4385) (end 142.975 88.8) (width 0.2) (layer "F.Cu") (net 2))
 (segment (start 142.09766 102.601) (end 145.6135 99.08516) (width 0.2) (layer "F.Cu") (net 2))
 (segment (start 128.8 103.315) (end 131.965 103.315) (width 0.2) (layer "F.Cu") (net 2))
 (segment (start 145.6135 94.28516) (end 145.6135 91.4385) (width 0.2) (layer "F.Cu") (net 2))
 (segment (start 132.65 100) (end 131.576 100) (width 0.2) (layer "F.Cu") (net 2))
 (segment (start 132.8 100) (end 132.65 100) (width 0.2) (layer "F.Cu") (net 2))
 (segment (start 131.576 100) (end 131.2 99.624) (width 0.2) (layer "F.Cu") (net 2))
 (segment (start 125.23 87.58) (end 125.732 87.078) (width 0.2) (layer "F.Cu") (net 2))
 (segment (start 137.6 102.46116) (end 135.03516 105.026) (width 0.2) (layer "F.Cu") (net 2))
 (segment (start 127.649 102.164) (end 128.8 103.315) (width 0.2) (layer "F.Cu") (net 2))
 (segment (start 145.6135 99.08516) (end 145.6135 96.2385) (width 0.2) (layer "F.Cu") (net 2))
 (segment (start 133.676 105.026) (end 132.65 104) (width 0.2) (layer "F.Cu") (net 2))
 (segment (start 145.29766 94.601) (end 145.6135 94.28516) (width 0.2) (layer "F.Cu") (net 2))
 (segment (start 143.976 94.601) (end 145.29766 94.601) (width 0.2) (layer "F.Cu") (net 2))
 (segment (start 135.03516 105.026) (end 133.676 105.026) (width 0.2) (layer "F.Cu") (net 2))
 (segment (start 137.6 101.6) (end 138.601 102.601) (width 0.2) (layer "F.Cu") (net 2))
 (segment (start 141.6 101.6) (end 144.8 98.4) (width 0.2) (layer "F.Cu") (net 3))
 (segment (start 139.475 101.6) (end 141.6 101.6) (width 0.2) (layer "F.Cu") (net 3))
 (segment (start 127.23 88.505) (end 127.23 88.77) (width 0.2) (layer "F.Cu") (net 4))
 (segment (start 127.23 89.482) (end 127.23 88.505) (width 0.2) (layer "F.Cu") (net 4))
 (segment (start 129.748 92) (end 127.23 89.482) (width 0.2) (layer "F.Cu") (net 4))
 (segment (start 144.8 93.6) (end 143.2 92) (width 0.2) (layer "F.Cu") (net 4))
 (segment (start 127.2 88.8) (end 127.23 88.77) (width 0.2) (layer "F.Cu") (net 4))
 (segment (start 143.2 92) (end 129.748 92) (width 0.2) (layer "F.Cu") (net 4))
 (segment (start 132.8 89.6) (end 132.8 89.42) (width 0.2) (layer "F.Cu") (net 10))
 (segment (start 124.16 93.6) (end 124.16 89.42) (width 0.2) (layer "F.Cu") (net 10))
 (segment (start 132.8 88.8) (end 132.8 89.42) (width 0.2) (layer "F.Cu") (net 10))
 (segment (start 144.8 88.8) (end 143.479 87.479) (width 0.2) (layer "F.Cu") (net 5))
 (segment (start 130.23 87.578) (end 130.23 88.505) (width 0.2) (layer "F.Cu") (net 5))
 (segment (start 143.479 87.479) (end 130.329 87.479) (width 0.2) (layer "F.Cu") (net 5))
 (segment (start 130.329 87.479) (end 130.23 87.578) (width 0.2) (layer "F.Cu") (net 5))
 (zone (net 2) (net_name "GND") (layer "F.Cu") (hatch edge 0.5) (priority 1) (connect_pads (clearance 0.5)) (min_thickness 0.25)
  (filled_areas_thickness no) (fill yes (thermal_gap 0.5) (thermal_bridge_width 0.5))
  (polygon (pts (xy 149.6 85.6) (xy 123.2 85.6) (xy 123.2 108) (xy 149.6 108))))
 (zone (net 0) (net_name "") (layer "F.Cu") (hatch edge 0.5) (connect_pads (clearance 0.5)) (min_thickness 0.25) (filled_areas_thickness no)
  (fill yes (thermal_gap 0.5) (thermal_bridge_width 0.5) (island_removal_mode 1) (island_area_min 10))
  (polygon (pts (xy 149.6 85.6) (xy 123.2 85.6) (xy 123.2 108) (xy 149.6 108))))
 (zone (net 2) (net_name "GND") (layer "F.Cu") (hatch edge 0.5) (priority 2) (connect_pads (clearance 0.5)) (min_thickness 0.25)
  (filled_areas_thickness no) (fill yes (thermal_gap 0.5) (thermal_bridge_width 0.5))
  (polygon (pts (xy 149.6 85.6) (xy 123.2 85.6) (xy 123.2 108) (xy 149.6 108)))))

